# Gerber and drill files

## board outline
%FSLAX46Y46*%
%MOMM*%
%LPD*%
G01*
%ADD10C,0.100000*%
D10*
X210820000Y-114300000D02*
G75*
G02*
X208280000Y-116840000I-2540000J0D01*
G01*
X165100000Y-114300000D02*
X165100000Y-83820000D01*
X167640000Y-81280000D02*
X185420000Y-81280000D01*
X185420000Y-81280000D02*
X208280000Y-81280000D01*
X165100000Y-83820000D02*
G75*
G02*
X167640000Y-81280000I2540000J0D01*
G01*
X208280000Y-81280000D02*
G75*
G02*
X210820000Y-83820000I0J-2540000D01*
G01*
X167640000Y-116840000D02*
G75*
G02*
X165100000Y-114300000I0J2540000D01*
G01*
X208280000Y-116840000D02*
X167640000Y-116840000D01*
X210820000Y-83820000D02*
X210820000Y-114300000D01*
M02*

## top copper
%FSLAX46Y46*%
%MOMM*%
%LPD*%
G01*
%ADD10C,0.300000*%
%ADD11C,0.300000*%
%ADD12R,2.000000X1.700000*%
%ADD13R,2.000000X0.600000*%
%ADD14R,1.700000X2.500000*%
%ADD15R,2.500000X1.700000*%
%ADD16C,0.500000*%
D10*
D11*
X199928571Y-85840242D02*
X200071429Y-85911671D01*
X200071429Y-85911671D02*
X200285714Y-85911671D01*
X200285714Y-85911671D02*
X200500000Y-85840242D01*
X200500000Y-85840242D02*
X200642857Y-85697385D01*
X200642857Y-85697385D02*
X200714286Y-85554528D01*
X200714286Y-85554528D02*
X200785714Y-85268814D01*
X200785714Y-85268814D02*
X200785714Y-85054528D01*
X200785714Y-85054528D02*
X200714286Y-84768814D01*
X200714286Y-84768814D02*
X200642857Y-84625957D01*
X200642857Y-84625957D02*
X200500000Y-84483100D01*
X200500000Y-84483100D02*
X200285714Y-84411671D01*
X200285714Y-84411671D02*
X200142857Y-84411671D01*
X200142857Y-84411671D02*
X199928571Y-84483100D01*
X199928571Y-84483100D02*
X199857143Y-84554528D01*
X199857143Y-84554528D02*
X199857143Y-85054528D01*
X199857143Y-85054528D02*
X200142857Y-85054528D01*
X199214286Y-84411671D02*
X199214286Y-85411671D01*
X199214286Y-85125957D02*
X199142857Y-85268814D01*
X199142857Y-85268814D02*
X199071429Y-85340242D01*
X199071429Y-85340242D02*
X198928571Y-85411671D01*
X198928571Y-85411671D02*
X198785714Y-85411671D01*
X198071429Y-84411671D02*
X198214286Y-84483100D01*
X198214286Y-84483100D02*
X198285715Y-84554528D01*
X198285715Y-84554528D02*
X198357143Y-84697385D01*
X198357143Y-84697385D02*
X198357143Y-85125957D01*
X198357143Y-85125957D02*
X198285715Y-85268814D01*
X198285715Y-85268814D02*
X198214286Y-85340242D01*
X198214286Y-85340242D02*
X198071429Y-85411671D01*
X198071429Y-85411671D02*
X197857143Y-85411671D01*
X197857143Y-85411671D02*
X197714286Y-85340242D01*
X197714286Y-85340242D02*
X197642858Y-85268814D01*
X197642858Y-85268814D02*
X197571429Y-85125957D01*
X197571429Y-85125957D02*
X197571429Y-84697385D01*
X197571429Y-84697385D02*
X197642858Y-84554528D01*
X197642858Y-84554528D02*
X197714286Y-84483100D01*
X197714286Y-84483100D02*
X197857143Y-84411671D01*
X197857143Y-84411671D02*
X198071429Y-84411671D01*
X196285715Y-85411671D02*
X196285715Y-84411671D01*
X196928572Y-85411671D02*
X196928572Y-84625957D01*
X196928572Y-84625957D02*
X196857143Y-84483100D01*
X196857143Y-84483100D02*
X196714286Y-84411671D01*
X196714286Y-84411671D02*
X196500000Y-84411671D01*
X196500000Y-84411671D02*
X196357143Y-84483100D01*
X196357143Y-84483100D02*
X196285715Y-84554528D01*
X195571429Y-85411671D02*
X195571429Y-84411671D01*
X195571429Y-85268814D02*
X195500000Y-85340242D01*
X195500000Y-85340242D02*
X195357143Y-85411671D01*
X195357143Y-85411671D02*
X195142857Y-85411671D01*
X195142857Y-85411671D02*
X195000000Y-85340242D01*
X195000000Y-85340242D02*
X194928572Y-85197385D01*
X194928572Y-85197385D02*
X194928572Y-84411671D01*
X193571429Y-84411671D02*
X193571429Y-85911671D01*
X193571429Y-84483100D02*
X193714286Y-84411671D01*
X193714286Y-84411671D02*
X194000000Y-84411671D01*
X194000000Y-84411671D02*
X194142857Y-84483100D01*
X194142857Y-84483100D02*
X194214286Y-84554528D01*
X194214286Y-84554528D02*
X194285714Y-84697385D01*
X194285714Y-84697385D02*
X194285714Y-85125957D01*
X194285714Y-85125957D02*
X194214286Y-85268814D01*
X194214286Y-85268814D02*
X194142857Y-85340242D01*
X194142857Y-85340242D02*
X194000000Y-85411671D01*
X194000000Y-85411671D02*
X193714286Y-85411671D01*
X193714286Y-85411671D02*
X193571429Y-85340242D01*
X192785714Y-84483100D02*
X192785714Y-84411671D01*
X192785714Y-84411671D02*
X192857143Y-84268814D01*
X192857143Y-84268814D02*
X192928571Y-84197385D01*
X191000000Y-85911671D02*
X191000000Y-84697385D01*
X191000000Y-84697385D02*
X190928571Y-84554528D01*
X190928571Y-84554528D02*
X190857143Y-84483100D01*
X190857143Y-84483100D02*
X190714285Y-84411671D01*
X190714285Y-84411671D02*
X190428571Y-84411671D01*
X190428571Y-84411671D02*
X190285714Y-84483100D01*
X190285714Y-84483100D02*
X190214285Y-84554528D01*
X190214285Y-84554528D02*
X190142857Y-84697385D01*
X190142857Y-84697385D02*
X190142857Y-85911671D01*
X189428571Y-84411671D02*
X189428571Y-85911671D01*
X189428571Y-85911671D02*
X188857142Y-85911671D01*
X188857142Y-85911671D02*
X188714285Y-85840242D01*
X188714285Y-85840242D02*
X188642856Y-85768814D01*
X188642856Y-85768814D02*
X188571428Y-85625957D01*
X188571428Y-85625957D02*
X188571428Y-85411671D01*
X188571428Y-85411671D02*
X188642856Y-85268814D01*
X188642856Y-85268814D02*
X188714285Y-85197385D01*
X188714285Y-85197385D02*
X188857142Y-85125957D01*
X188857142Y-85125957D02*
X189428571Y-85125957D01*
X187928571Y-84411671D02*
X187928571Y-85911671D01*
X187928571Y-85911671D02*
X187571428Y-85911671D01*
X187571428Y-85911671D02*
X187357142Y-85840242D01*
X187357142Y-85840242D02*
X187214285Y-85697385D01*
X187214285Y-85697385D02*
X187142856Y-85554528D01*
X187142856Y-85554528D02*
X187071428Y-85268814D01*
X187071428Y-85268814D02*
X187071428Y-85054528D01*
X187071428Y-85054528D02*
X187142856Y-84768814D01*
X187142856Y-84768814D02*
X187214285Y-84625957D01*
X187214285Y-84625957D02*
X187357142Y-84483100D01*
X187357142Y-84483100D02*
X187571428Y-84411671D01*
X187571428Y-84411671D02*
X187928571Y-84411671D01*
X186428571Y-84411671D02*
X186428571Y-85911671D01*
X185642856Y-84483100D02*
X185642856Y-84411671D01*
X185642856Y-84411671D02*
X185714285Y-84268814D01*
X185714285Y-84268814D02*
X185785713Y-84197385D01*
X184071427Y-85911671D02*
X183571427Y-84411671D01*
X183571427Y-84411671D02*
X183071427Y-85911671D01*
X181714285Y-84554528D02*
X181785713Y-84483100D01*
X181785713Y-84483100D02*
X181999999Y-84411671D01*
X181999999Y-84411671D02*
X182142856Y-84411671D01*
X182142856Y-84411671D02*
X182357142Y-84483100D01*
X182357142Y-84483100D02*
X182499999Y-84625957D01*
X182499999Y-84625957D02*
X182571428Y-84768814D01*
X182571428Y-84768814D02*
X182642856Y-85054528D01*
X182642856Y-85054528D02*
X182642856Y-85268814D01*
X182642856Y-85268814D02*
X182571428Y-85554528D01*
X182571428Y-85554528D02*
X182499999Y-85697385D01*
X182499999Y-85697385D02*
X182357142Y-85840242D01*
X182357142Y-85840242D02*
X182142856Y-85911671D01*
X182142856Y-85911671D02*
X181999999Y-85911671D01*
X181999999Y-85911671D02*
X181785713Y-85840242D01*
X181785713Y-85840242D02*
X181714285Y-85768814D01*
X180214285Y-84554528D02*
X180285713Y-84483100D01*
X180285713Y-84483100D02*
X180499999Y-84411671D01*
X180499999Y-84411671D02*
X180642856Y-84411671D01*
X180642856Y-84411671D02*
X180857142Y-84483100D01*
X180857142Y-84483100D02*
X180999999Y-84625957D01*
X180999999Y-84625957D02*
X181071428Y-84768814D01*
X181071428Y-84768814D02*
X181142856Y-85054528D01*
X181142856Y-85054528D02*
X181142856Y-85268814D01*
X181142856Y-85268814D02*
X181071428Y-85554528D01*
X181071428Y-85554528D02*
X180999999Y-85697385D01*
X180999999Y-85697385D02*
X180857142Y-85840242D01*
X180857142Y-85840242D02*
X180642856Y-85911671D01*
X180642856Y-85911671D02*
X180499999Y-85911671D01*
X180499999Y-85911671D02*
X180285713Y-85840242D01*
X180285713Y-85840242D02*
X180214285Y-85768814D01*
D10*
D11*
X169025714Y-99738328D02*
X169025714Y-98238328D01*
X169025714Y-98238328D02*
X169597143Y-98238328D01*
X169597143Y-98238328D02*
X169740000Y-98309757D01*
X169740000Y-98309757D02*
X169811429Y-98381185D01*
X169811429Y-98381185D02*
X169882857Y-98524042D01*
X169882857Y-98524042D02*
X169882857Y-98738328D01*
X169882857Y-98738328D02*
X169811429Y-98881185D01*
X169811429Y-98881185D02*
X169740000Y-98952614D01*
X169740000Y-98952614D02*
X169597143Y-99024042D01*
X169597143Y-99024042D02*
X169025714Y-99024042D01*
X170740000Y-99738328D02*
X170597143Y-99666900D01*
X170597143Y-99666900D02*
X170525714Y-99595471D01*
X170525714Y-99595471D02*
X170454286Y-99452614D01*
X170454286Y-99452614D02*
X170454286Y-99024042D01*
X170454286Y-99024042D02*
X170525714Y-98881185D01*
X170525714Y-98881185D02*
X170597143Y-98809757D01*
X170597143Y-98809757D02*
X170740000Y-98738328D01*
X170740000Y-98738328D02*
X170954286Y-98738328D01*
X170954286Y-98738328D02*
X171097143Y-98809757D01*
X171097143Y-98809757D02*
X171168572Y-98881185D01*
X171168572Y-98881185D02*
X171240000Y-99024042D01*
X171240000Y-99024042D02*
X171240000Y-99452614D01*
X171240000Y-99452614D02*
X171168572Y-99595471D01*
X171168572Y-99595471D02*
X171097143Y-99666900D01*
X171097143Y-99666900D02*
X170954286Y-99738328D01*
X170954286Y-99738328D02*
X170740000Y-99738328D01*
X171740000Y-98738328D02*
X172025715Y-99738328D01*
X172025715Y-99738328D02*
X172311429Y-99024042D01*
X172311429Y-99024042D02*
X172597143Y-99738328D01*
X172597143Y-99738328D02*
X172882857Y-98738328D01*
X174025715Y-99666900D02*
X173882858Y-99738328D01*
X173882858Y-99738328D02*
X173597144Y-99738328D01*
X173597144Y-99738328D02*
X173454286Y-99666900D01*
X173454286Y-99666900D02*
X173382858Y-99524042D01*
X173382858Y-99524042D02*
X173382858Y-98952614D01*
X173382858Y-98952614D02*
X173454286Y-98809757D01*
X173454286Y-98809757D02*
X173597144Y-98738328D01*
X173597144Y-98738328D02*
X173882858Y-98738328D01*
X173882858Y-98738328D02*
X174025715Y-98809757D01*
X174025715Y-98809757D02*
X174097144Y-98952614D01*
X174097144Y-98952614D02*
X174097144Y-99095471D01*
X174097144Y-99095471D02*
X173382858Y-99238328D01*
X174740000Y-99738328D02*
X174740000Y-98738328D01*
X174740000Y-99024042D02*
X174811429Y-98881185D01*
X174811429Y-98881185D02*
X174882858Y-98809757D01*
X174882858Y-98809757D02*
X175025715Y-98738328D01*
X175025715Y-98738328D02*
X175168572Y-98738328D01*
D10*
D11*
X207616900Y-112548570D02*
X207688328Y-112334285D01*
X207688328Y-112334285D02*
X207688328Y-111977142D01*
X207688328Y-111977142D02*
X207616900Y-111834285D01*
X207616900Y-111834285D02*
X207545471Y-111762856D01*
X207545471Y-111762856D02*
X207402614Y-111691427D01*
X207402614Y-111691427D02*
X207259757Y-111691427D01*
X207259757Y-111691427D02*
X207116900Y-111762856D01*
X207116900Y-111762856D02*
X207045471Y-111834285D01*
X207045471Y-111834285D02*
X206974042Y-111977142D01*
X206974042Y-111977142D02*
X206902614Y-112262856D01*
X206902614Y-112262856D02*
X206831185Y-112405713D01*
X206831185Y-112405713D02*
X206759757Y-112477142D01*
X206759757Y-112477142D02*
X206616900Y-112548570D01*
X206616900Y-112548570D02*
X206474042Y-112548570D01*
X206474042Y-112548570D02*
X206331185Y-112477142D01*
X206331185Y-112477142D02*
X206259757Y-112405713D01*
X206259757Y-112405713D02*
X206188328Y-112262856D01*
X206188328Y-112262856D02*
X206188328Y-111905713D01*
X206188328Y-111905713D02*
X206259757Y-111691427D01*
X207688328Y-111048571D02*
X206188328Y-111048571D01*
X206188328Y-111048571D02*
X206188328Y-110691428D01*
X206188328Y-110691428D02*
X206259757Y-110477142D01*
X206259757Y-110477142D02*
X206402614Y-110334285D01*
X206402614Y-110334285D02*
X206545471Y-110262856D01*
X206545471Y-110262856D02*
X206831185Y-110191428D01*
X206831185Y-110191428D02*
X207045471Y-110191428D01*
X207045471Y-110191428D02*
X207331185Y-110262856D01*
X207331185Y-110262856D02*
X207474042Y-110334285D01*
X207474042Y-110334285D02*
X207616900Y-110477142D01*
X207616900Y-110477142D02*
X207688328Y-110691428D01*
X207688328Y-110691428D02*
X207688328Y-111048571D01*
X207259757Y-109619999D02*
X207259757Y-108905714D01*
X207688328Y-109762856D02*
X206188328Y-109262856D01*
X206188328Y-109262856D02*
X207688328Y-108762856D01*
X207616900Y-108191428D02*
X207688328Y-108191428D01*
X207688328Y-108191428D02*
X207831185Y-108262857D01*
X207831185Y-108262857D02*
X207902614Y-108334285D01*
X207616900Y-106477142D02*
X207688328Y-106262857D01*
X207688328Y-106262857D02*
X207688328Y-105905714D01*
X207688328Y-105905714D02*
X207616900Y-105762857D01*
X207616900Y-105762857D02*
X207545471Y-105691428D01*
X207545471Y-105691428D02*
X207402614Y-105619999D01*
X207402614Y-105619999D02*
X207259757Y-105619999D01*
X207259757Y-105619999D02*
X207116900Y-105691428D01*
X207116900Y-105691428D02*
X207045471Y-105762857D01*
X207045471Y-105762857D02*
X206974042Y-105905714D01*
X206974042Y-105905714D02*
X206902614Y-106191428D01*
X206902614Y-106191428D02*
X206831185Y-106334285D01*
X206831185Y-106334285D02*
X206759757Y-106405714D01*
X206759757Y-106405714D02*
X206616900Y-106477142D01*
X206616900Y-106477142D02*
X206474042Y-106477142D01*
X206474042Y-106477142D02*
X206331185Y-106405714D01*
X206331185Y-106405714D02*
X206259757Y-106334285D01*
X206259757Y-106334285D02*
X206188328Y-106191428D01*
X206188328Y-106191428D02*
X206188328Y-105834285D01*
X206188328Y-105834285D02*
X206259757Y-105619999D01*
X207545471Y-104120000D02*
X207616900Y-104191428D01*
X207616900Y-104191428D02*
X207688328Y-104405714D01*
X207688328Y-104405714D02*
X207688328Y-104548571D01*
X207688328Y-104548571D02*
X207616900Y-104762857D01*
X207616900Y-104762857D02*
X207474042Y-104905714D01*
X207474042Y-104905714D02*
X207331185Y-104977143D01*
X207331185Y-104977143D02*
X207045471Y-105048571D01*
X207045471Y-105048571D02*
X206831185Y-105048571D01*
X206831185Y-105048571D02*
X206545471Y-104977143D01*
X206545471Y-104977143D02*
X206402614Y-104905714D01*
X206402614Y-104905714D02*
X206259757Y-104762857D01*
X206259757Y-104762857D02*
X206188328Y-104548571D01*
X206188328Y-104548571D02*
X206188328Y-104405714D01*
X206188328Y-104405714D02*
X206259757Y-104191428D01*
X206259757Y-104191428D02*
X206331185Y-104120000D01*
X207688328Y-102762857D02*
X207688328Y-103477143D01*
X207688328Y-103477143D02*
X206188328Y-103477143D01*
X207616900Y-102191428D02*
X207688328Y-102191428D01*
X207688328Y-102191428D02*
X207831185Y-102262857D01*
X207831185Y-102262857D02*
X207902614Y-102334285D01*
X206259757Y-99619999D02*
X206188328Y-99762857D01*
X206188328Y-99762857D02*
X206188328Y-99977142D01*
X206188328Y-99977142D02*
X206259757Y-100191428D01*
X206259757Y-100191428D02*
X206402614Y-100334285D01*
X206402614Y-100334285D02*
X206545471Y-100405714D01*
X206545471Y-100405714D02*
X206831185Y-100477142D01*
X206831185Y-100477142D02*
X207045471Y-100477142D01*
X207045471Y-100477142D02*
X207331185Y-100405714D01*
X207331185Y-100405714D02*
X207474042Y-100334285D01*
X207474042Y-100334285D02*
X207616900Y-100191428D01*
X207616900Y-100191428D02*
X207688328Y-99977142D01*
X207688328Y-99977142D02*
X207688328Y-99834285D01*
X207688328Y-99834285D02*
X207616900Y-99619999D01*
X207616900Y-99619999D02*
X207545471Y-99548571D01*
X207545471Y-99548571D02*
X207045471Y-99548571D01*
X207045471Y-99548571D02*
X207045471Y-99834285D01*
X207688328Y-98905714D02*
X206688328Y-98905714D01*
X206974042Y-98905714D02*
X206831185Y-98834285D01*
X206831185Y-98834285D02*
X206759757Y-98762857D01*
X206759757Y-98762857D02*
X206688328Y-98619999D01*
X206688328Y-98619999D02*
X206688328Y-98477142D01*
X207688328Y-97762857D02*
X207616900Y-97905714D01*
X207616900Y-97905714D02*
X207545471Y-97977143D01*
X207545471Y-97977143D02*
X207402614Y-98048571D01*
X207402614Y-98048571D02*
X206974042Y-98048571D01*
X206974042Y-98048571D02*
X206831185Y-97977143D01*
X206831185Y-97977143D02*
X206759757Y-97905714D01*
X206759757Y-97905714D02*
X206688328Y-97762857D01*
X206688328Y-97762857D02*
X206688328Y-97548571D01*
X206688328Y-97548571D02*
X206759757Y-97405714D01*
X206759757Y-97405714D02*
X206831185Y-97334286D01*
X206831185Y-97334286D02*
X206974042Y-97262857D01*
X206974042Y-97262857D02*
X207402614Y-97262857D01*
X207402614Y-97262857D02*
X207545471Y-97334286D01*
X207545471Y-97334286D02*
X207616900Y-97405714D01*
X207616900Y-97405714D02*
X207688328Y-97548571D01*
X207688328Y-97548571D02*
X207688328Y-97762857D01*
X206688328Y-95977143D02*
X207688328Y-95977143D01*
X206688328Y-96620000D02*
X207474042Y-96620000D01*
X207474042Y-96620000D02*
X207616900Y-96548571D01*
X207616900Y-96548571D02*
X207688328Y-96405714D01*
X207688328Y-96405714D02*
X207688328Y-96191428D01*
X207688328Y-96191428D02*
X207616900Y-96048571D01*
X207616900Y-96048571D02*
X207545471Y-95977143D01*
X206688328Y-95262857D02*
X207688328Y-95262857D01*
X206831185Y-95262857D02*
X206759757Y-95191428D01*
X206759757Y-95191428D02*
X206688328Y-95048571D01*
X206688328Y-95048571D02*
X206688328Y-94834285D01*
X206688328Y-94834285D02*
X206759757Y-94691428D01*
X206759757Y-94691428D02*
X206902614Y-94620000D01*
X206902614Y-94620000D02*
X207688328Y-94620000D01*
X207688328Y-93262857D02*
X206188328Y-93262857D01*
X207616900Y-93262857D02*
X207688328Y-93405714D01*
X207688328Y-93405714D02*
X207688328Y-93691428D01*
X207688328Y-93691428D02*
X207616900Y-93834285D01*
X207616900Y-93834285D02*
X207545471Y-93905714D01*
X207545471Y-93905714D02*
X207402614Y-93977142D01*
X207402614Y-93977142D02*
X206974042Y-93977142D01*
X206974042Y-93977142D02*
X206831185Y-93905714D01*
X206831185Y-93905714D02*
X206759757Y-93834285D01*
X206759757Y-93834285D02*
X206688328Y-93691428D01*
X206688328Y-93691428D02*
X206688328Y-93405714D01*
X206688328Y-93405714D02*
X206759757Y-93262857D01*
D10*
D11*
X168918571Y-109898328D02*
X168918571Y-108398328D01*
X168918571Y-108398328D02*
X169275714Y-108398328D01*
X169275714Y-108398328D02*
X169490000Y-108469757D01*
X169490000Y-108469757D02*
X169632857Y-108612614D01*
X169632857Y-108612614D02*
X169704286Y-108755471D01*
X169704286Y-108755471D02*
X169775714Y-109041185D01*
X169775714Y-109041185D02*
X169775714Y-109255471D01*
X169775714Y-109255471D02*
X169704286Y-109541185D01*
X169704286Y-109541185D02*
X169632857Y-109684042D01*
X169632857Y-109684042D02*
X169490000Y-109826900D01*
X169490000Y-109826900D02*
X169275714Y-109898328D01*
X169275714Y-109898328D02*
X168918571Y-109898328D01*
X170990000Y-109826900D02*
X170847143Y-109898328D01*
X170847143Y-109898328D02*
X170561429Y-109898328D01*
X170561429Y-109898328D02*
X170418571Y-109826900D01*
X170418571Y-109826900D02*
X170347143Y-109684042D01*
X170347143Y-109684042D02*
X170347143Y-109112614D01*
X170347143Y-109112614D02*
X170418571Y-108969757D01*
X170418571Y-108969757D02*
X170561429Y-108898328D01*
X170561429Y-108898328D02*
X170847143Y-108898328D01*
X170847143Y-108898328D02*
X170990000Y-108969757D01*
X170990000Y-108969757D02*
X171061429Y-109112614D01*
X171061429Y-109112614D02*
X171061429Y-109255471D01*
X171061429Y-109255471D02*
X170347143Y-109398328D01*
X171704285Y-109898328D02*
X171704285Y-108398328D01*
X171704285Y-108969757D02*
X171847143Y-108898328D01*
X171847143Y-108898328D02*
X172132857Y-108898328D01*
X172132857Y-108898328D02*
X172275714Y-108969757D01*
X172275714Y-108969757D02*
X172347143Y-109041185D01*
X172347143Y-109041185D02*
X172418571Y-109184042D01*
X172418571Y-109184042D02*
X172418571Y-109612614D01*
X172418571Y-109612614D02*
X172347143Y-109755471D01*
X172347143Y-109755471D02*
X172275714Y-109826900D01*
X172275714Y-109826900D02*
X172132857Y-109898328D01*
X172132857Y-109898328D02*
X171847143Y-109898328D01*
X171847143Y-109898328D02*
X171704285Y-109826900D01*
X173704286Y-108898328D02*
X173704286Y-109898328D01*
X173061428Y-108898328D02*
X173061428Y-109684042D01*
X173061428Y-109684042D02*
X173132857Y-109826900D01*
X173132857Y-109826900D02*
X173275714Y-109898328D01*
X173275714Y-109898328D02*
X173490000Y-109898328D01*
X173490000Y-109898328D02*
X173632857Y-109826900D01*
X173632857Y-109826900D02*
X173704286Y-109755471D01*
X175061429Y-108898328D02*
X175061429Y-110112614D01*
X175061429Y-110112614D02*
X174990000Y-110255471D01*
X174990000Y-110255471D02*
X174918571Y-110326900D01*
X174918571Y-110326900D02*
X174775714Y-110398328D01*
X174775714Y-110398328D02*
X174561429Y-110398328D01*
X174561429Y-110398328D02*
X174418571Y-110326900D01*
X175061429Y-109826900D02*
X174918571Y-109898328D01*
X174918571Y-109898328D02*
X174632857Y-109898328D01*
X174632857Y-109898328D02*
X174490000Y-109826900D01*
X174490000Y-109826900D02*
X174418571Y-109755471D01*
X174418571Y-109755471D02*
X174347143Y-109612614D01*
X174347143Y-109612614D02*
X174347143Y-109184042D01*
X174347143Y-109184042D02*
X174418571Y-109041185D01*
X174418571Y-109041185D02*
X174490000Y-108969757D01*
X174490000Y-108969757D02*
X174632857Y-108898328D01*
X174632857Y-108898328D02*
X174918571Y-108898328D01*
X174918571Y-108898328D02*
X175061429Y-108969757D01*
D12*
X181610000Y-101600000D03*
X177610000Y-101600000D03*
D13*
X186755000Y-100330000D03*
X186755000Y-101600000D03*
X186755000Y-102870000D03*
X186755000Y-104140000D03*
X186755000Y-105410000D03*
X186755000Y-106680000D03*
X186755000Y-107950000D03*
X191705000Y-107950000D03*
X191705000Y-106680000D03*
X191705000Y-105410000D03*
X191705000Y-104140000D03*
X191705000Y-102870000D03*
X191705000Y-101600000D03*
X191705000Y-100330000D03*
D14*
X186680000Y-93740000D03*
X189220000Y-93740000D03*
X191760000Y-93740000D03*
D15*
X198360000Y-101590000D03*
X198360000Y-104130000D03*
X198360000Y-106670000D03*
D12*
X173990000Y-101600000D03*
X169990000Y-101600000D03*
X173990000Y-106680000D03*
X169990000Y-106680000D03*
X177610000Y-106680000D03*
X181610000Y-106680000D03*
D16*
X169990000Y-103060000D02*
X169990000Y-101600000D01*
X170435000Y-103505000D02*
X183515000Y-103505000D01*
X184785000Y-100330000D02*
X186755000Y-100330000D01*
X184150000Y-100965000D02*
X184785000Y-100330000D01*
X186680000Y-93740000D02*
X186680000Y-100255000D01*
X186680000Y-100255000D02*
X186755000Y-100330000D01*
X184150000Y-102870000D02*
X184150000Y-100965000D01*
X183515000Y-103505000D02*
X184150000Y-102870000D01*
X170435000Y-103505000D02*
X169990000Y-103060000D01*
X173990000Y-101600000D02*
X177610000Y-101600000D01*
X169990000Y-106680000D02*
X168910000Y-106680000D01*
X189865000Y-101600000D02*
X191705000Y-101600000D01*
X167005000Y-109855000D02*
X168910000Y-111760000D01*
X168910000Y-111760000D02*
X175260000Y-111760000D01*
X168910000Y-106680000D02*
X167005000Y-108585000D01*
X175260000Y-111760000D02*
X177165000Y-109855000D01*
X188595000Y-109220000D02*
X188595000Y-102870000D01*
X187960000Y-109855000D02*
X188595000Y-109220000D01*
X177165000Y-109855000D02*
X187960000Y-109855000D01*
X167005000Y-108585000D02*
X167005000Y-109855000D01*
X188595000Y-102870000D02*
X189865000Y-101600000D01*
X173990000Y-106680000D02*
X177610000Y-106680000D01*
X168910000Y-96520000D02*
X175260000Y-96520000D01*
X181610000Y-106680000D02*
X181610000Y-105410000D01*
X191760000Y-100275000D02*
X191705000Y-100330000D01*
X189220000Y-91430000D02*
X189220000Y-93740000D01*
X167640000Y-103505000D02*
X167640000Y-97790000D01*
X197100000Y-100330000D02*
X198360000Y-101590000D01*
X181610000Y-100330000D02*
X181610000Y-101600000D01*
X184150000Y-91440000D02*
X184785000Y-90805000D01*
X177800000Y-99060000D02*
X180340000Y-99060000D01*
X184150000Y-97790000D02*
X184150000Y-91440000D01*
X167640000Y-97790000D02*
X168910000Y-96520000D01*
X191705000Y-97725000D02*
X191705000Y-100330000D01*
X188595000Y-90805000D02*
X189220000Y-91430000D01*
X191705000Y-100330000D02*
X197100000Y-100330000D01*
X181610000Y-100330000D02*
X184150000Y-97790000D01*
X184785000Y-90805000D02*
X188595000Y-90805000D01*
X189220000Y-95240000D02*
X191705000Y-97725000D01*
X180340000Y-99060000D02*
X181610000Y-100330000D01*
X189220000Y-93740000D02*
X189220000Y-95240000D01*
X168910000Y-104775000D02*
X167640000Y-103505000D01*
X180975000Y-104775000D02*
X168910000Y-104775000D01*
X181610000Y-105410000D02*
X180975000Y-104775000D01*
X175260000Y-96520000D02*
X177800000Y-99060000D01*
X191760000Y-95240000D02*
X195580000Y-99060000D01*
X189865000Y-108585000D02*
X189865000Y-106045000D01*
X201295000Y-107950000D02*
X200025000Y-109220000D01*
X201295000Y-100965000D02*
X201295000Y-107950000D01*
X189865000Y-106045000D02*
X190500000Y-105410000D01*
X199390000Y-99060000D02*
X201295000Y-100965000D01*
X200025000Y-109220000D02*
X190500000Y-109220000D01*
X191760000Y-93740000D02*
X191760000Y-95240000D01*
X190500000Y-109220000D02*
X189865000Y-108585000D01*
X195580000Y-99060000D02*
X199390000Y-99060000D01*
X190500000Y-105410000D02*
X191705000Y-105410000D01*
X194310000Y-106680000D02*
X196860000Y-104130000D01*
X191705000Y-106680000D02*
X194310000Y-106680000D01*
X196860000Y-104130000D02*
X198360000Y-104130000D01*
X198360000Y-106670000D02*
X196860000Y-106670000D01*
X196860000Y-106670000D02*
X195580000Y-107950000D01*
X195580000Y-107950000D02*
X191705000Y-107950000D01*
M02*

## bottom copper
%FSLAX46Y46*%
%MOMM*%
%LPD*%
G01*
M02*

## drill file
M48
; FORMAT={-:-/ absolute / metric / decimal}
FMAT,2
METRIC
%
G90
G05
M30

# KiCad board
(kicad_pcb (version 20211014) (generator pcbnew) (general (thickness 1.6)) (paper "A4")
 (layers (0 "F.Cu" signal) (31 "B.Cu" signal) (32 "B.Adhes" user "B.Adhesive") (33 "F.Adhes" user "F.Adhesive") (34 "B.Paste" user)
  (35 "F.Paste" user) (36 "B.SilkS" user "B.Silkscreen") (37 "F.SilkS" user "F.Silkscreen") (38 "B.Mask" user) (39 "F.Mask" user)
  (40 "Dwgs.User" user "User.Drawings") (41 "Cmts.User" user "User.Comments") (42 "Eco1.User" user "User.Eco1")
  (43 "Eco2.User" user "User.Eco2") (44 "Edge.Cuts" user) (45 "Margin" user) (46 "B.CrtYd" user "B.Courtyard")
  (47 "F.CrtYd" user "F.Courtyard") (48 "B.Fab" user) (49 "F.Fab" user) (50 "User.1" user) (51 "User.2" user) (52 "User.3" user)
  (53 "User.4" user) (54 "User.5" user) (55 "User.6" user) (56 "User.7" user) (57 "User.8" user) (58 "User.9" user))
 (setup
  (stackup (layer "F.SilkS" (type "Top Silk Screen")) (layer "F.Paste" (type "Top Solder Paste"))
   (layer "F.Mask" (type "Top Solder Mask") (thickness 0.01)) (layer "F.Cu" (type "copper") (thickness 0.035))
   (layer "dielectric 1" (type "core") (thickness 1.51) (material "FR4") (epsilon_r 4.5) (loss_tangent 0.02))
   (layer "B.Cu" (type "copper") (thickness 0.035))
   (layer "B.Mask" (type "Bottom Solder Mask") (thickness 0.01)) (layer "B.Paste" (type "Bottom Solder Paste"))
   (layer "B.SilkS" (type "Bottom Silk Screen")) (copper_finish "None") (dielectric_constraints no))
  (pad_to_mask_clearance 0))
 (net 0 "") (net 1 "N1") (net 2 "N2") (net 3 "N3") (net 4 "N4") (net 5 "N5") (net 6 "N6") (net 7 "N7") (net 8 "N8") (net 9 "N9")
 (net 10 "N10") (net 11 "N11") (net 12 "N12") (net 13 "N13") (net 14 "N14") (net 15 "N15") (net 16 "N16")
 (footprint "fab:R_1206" (layer "F.Cu") (at 179.61 101.6 180)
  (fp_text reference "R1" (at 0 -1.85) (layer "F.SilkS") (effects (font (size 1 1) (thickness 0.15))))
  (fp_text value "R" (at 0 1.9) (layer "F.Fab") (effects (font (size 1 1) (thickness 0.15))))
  (pad "1" smd rect locked (at -2 0 180) (size 2 1.7) (layers "F.Cu" "F.Paste" "F.Mask") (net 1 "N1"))
  (pad "2" smd rect locked (at 2 0 180) (size 2 1.7) (layers "F.Cu" "F.Paste" "F.Mask") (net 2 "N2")))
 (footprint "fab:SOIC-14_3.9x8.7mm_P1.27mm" (layer "F.Cu") (at 189.23 104.14)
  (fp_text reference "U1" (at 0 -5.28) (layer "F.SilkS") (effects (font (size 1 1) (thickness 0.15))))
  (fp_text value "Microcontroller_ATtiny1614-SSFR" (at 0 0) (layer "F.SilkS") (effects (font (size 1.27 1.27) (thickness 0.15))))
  (pad "1" smd rect (at -2.475 -3.81) (size 2 0.6) (layers "F.Cu" "F.Paste" "F.Mask") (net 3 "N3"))
  (pad "2" smd rect (at -2.475 -2.54) (size 2 0.6) (layers "F.Cu" "F.Paste" "F.Mask") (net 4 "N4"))
  (pad "3" smd rect (at -2.475 -1.27) (size 2 0.6) (layers "F.Cu" "F.Paste" "F.Mask") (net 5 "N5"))
  (pad "4" smd rect (at -2.475 0) (size 2 0.6) (layers "F.Cu" "F.Paste" "F.Mask") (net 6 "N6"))
  (pad "5" smd rect (at -2.475 1.27) (size 2 0.6) (layers "F.Cu" "F.Paste" "F.Mask") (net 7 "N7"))
  (pad "6" smd rect (at -2.475 2.54) (size 2 0.6) (layers "F.Cu" "F.Paste" "F.Mask") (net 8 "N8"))
  (pad "7" smd rect (at -2.475 3.81) (size 2 0.6) (layers "F.Cu" "F.Paste" "F.Mask") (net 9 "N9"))
  (pad "8" smd rect (at 2.475 3.81) (size 2 0.6) (layers "F.Cu" "F.Paste" "F.Mask") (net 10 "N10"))
  (pad "9" smd rect (at 2.475 2.54) (size 2 0.6) (layers "F.Cu" "F.Paste" "F.Mask") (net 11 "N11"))
  (pad "10" smd rect (at 2.475 1.27) (size 2 0.6) (layers "F.Cu" "F.Paste" "F.Mask") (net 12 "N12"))
  (pad "11" smd rect (at 2.475 0) (size 2 0.6) (layers "F.Cu" "F.Paste" "F.Mask") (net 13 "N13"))
  (pad "12" smd rect (at 2.475 -1.27) (size 2 0.6) (layers "F.Cu" "F.Paste" "F.Mask") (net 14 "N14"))
  (pad "13" smd rect (at 2.475 -2.54) (size 2 0.6) (layers "F.Cu" "F.Paste" "F.Mask") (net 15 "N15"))
  (pad "14" smd rect (at 2.475 -3.81) (size 2 0.6) (layers "F.Cu" "F.Paste" "F.Mask") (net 1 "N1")))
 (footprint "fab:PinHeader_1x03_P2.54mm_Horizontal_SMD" (layer "F.Cu") (at 186.68 93.74 90)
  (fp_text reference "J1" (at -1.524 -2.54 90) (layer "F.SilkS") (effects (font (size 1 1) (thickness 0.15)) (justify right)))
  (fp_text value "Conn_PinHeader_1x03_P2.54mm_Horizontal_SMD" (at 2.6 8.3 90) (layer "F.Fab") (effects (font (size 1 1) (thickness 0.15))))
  (pad "1" smd rect locked (at 0 0 90) (size 2.5 1.7) (layers "F.Cu" "F.Paste" "F.Mask") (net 3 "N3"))
  (pad "2" smd rect locked (at 0 2.54 90) (size 2.5 1.7) (layers "F.Cu" "F.Paste" "F.Mask") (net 1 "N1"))
  (pad "3" smd rect locked (at 0 5.08 90) (size 2.5 1.7) (layers "F.Cu" "F.Paste" "F.Mask") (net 12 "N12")))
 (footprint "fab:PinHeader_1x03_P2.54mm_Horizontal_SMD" (layer "F.Cu") (at 198.36 101.59)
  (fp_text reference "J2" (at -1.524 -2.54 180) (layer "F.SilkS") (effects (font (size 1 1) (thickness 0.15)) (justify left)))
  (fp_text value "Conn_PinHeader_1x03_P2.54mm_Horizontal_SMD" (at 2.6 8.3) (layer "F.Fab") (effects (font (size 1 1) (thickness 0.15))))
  (pad "1" smd rect locked (at 0 0) (size 2.5 1.7) (layers "F.Cu" "F.Paste" "F.Mask") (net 1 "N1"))
  (pad "2" smd rect locked (at 0 2.54) (size 2.5 1.7) (layers "F.Cu" "F.Paste" "F.Mask") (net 11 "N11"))
  (pad "3" smd rect locked (at 0 5.08) (size 2.5 1.7) (layers "F.Cu" "F.Paste" "F.Mask") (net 10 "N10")))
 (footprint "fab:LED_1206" (layer "F.Cu") (at 171.99 101.6 180)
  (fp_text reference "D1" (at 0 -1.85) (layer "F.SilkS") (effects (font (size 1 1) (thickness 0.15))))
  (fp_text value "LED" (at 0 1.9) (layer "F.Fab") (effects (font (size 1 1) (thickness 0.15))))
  (pad "1" smd rect locked (at -2 0 180) (size 2 1.7) (layers "F.Cu" "F.Paste" "F.Mask") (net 2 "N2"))
  (pad "2" smd rect locked (at 2 0 180) (size 2 1.7) (layers "F.Cu" "F.Paste" "F.Mask") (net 3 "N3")))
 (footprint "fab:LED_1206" (layer "F.Cu") (at 171.99 106.68 180)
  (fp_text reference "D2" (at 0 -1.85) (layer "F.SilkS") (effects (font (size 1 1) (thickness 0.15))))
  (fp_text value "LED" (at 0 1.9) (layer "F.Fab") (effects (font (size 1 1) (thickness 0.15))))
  (pad "1" smd rect locked (at -2 0 180) (size 2 1.7) (layers "F.Cu" "F.Paste" "F.Mask") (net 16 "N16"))
  (pad "2" smd rect locked (at 2 0 180) (size 2 1.7) (layers "F.Cu" "F.Paste" "F.Mask") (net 15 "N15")))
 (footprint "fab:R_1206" (layer "F.Cu") (at 179.61 106.68)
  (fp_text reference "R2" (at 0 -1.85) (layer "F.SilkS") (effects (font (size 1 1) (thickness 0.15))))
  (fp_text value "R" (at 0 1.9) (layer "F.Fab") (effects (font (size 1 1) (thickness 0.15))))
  (pad "1" smd rect locked (at -2 0) (size 2 1.7) (layers "F.Cu" "F.Paste" "F.Mask") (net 16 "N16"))
  (pad "2" smd rect locked (at 2 0) (size 2 1.7) (layers "F.Cu" "F.Paste" "F.Mask") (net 1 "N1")))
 (gr_arc (start 210.82 114.3) (mid 210.076051 116.096051) (end 208.28 116.84) (layer "Edge.Cuts") (width 0.1))
 (gr_line (start 165.1 114.3) (end 165.1 83.82) (layer "Edge.Cuts") (width 0.1))
 (gr_line (start 167.64 81.28) (end 185.42 81.28) (layer "Edge.Cuts") (width 0.1))
 (gr_line (start 185.42 81.28) (end 208.28 81.28) (layer "Edge.Cuts") (width 0.1))
 (gr_arc (start 165.1 83.82) (mid 165.843949 82.023949) (end 167.64 81.28) (layer "Edge.Cuts") (width 0.1))
 (gr_arc (start 208.28 81.28) (mid 210.076051 82.023949) (end 210.82 83.82) (layer "Edge.Cuts") (width 0.1))
 (gr_arc (start 167.64 116.84) (mid 165.843949 116.096051) (end 165.1 114.3) (layer "Edge.Cuts") (width 0.1))
 (gr_line (start 208.28 116.84) (end 167.64 116.84) (layer "Edge.Cuts") (width 0.1))
 (gr_line (start 210.82 83.82) (end 210.82 114.3) (layer "Edge.Cuts") (width 0.1))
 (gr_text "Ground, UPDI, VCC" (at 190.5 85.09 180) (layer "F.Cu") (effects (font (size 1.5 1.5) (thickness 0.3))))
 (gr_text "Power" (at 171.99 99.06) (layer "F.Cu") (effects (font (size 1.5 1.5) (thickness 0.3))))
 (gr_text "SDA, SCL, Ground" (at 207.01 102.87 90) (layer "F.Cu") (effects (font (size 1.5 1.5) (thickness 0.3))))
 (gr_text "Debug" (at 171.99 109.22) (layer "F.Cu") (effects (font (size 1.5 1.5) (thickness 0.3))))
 (segment (start 169.99 103.06) (end 169.99 101.6) (width 0.5) (layer "F.Cu") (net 3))
 (segment (start 170.435 103.505) (end 183.515 103.505) (width 0.5) (layer "F.Cu") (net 3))
 (segment (start 184.785 100.33) (end 186.755 100.33) (width 0.5) (layer "F.Cu") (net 3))
 (segment (start 184.15 100.965) (end 184.785 100.33) (width 0.5) (layer "F.Cu") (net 3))
 (segment (start 186.68 93.74) (end 186.68 100.255) (width 0.5) (layer "F.Cu") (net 3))
 (segment (start 186.68 100.255) (end 186.755 100.33) (width 0.5) (layer "F.Cu") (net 3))
 (segment (start 184.15 102.87) (end 184.15 100.965) (width 0.5) (layer "F.Cu") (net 3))
 (segment (start 183.515 103.505) (end 184.15 102.87) (width 0.5) (layer "F.Cu") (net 3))
 (segment (start 170.435 103.505) (end 169.99 103.06) (width 0.5) (layer "F.Cu") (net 3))
 (segment (start 173.99 101.6) (end 177.61 101.6) (width 0.5) (layer "F.Cu") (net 2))
 (segment (start 169.99 106.68) (end 168.91 106.68) (width 0.5) (layer "F.Cu") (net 15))
 (segment (start 189.865 101.6) (end 191.705 101.6) (width 0.5) (layer "F.Cu") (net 15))
 (segment (start 167.005 109.855) (end 168.91 111.76) (width 0.5) (layer "F.Cu") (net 15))
 (segment (start 168.91 111.76) (end 175.26 111.76) (width 0.5) (layer "F.Cu") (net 15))
 (segment (start 168.91 106.68) (end 167.005 108.585) (width 0.5) (layer "F.Cu") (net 15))
 (segment (start 175.26 111.76) (end 177.165 109.855) (width 0.5) (layer "F.Cu") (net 15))
 (segment (start 188.595 109.22) (end 188.595 102.87) (width 0.5) (layer "F.Cu") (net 15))
 (segment (start 187.96 109.855) (end 188.595 109.22) (width 0.5) (layer "F.Cu") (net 15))
 (segment (start 177.165 109.855) (end 187.96 109.855) (width 0.5) (layer "F.Cu") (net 15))
 (segment (start 167.005 108.585) (end 167.005 109.855) (width 0.5) (layer "F.Cu") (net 15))
 (segment (start 188.595 102.87) (end 189.865 101.6) (width 0.5) (layer "F.Cu") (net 15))
 (segment (start 173.99 106.68) (end 177.61 106.68) (width 0.5) (layer "F.Cu") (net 16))
 (segment (start 168.91 96.52) (end 175.26 96.52) (width 0.5) (layer "F.Cu") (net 1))
 (segment (start 181.61 106.68) (end 181.61 105.41) (width 0.5) (layer "F.Cu") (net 1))
 (segment (start 191.76 100.275) (end 191.705 100.33) (width 0.5) (layer "F.Cu") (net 1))
 (segment (start 189.22 91.43) (end 189.22 93.74) (width 0.5) (layer "F.Cu") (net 1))
 (segment (start 167.64 103.505) (end 167.64 97.79) (width 0.5) (layer "F.Cu") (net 1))
 (segment (start 197.1 100.33) (end 198.36 101.59) (width 0.5) (layer "F.Cu") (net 1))
 (segment (start 181.61 100.33) (end 181.61 101.6) (width 0.5) (layer "F.Cu") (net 1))
 (segment (start 184.15 91.44) (end 184.785 90.805) (width 0.5) (layer "F.Cu") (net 1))
 (segment (start 177.8 99.06) (end 180.34 99.06) (width 0.5) (layer "F.Cu") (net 1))
 (segment (start 184.15 97.79) (end 184.15 91.44) (width 0.5) (layer "F.Cu") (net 1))
 (segment (start 167.64 97.79) (end 168.91 96.52) (width 0.5) (layer "F.Cu") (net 1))
 (segment (start 191.705 97.725) (end 191.705 100.33) (width 0.5) (layer "F.Cu") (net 1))
 (segment (start 188.595 90.805) (end 189.22 91.43) (width 0.5) (layer "F.Cu") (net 1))
 (segment (start 191.705 100.33) (end 197.1 100.33) (width 0.5) (layer "F.Cu") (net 1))
 (segment (start 181.61 100.33) (end 184.15 97.79) (width 0.5) (layer "F.Cu") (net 1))
 (segment (start 184.785 90.805) (end 188.595 90.805) (width 0.5) (layer "F.Cu") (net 1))
 (segment (start 189.22 95.24) (end 191.705 97.725) (width 0.5) (layer "F.Cu") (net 1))
 (segment (start 180.34 99.06) (end 181.61 100.33) (width 0.5) (layer "F.Cu") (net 1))
 (segment (start 189.22 93.74) (end 189.22 95.24) (width 0.5) (layer "F.Cu") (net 1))
 (segment (start 168.91 104.775) (end 167.64 103.505) (width 0.5) (layer "F.Cu") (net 1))
 (segment (start 180.975 104.775) (end 168.91 104.775) (width 0.5) (layer "F.Cu") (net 1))
 (segment (start 181.61 105.41) (end 180.975 104.775) (width 0.5) (layer "F.Cu") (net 1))
 (segment (start 175.26 96.52) (end 177.8 99.06) (width 0.5) (layer "F.Cu") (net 1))
 (segment (start 191.76 95.24) (end 195.58 99.06) (width 0.5) (layer "F.Cu") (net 12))
 (segment (start 189.865 108.585) (end 189.865 106.045) (width 0.5) (layer "F.Cu") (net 12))
 (segment (start 201.295 107.95) (end 200.025 109.22) (width 0.5) (layer "F.Cu") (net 12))
 (segment (start 201.295 100.965) (end 201.295 107.95) (width 0.5) (layer "F.Cu") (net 12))
 (segment (start 189.865 106.045) (end 190.5 105.41) (width 0.5) (layer "F.Cu") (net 12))
 (segment (start 199.39 99.06) (end 201.295 100.965) (width 0.5) (layer "F.Cu") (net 12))
 (segment (start 200.025 109.22) (end 190.5 109.22) (width 0.5) (layer "F.Cu") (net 12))
 (segment (start 191.76 93.74) (end 191.76 95.24) (width 0.5) (layer "F.Cu") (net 12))
 (segment (start 190.5 109.22) (end 189.865 108.585) (width 0.5) (layer "F.Cu") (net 12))
 (segment (start 195.58 99.06) (end 199.39 99.06) (width 0.5) (layer "F.Cu") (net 12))
 (segment (start 190.5 105.41) (end 191.705 105.41) (width 0.5) (layer "F.Cu") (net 12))
 (segment (start 194.31 106.68) (end 196.86 104.13) (width 0.5) (layer "F.Cu") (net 11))
 (segment (start 191.705 106.68) (end 194.31 106.68) (width 0.5) (layer "F.Cu") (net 11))
 (segment (start 196.86 104.13) (end 198.36 104.13) (width 0.5) (layer "F.Cu") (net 11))
 (segment (start 198.36 106.67) (end 196.86 106.67) (width 0.5) (layer "F.Cu") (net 10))
 (segment (start 196.86 106.67) (end 195.58 107.95) (width 0.5) (layer "F.Cu") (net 10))
 (segment (start 195.58 107.95) (end 191.705 107.95) (width 0.5) (layer "F.Cu") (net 10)))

